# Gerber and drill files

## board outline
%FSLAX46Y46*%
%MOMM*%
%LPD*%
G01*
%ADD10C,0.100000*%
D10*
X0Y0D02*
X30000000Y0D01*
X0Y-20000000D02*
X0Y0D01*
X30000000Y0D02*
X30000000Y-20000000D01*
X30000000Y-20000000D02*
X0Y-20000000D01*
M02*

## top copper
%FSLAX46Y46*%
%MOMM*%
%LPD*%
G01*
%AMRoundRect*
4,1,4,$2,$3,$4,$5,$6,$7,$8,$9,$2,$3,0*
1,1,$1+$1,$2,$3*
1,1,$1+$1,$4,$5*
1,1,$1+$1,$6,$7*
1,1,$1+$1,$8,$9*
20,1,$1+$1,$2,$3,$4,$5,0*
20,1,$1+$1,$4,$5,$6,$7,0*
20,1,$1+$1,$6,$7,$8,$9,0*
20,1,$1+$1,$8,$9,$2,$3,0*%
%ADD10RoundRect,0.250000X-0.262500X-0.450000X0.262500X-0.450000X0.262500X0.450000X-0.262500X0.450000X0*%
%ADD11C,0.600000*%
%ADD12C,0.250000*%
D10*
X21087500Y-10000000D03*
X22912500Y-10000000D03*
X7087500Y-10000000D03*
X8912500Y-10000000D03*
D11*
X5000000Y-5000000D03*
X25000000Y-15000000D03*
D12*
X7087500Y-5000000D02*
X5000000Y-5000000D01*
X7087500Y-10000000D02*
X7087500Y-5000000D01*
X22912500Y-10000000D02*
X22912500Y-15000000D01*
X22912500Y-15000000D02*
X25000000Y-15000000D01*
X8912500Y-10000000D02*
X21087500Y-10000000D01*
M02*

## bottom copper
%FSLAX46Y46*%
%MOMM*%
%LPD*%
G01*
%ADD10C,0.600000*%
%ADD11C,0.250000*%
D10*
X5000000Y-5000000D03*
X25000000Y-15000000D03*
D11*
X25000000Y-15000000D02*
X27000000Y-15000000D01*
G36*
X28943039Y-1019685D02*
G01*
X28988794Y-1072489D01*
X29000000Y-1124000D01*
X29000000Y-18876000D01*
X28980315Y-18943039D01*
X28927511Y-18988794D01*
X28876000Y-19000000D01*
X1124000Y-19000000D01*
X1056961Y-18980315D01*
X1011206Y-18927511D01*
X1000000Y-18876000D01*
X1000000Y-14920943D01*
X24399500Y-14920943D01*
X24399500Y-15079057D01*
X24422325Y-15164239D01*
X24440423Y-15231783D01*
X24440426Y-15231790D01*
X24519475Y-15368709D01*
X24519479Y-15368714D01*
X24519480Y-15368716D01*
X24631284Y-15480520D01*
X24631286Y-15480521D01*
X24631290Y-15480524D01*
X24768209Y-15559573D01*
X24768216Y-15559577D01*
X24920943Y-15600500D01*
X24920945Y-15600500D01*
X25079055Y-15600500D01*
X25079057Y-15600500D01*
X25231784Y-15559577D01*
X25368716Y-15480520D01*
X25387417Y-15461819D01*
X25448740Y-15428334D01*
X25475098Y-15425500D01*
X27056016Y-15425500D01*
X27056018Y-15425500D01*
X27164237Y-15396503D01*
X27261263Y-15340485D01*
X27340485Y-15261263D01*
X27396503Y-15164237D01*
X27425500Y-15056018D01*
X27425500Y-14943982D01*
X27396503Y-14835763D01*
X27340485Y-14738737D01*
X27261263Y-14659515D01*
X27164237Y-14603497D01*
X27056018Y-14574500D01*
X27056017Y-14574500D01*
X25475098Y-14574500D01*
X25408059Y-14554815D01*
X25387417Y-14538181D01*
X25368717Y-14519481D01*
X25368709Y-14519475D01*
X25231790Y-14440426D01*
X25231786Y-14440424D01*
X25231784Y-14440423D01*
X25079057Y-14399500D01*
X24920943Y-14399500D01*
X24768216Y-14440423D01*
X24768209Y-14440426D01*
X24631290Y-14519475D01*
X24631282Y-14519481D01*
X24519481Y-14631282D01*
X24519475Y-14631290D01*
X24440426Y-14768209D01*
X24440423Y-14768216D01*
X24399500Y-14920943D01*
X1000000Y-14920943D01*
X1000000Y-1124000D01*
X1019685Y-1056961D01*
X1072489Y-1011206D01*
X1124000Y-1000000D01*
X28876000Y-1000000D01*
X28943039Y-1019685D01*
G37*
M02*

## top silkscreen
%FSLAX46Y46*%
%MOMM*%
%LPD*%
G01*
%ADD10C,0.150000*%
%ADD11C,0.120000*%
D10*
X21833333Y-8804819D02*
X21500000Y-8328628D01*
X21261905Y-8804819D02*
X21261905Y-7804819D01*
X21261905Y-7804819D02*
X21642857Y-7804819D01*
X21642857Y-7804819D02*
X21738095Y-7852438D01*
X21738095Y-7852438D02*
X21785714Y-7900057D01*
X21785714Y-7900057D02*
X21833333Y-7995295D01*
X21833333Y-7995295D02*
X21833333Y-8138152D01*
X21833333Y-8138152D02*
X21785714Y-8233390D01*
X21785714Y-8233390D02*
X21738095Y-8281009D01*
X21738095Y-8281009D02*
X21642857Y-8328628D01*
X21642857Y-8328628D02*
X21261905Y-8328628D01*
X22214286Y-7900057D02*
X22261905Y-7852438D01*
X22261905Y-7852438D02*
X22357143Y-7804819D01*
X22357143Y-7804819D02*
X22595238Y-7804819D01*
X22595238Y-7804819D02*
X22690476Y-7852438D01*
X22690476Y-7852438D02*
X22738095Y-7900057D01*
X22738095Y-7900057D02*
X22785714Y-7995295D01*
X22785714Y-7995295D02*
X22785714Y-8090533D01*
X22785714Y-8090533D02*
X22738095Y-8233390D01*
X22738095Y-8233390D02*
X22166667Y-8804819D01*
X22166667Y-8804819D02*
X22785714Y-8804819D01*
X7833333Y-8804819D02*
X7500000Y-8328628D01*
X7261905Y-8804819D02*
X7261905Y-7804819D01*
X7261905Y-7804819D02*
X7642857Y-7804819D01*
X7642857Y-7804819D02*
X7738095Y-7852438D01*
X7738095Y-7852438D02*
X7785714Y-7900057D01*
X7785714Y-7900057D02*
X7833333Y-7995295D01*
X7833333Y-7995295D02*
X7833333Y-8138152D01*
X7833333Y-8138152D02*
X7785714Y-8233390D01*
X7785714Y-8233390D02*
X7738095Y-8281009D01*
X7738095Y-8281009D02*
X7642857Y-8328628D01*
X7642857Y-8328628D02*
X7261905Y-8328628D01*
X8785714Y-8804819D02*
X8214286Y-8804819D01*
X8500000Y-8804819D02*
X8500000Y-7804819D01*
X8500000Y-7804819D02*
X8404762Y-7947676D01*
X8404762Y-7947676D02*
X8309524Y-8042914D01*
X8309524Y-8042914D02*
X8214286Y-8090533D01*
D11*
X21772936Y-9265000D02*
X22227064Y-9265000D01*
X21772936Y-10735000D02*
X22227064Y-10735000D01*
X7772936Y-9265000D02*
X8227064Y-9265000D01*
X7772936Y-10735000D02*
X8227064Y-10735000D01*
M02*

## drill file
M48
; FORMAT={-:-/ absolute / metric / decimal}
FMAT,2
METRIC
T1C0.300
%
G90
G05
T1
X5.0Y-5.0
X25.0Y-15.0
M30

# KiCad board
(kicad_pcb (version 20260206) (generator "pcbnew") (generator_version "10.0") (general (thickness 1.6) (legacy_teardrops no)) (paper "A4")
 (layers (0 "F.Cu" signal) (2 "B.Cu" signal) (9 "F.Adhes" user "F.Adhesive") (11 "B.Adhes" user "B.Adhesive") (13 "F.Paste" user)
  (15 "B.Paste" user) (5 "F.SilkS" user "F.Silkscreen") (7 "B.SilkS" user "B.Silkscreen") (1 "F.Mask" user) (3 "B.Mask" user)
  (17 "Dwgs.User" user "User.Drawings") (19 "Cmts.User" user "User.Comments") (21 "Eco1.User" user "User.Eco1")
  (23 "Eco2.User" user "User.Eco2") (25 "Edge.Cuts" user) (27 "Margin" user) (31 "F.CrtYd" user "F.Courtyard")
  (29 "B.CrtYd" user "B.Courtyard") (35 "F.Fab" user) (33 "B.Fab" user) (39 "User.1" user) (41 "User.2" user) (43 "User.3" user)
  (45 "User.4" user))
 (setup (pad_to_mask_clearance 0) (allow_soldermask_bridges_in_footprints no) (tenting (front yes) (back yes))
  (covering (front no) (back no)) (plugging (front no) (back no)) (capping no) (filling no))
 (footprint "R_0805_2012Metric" (layer "F.Cu") (at 22 10)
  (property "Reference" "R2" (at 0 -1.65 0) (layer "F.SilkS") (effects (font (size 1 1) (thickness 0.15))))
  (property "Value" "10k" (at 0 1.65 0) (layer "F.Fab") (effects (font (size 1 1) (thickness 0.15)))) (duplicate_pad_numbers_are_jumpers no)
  (fp_line (start -0.227064 -0.735) (end 0.227064 -0.735) (stroke (width 0.12) (type solid)) (layer "F.SilkS"))
  (fp_line (start -0.227064 0.735) (end 0.227064 0.735) (stroke (width 0.12) (type solid)) (layer "F.SilkS"))
  (pad "1" smd roundrect (at -0.9125 0) (size 1.025 1.4) (layers "F.Cu" "F.Mask" "F.Paste") (roundrect_rratio 0.243902) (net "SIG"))
  (pad "2" smd roundrect (at 0.9125 0) (size 1.025 1.4) (layers "F.Cu" "F.Mask" "F.Paste") (roundrect_rratio 0.243902) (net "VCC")))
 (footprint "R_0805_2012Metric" (layer "F.Cu") (at 8 10)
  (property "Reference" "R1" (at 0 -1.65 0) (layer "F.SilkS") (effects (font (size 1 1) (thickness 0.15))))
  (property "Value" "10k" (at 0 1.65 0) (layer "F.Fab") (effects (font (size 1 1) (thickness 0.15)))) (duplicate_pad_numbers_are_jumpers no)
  (fp_line (start -0.227064 -0.735) (end 0.227064 -0.735) (stroke (width 0.12) (type solid)) (layer "F.SilkS"))
  (fp_line (start -0.227064 0.735) (end 0.227064 0.735) (stroke (width 0.12) (type solid)) (layer "F.SilkS"))
  (pad "1" smd roundrect (at -0.9125 0) (size 1.025 1.4) (layers "F.Cu" "F.Mask" "F.Paste") (roundrect_rratio 0.243902) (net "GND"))
  (pad "2" smd roundrect (at 0.9125 0) (size 1.025 1.4) (layers "F.Cu" "F.Mask" "F.Paste") (roundrect_rratio 0.243902) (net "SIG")))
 (gr_line (start 0 0) (end 30 0) (stroke (width 0.1) (type default)) (layer "Edge.Cuts"))
 (gr_line (start 0 20) (end 0 0) (stroke (width 0.1) (type default)) (layer "Edge.Cuts"))
 (gr_line (start 30 0) (end 30 20) (stroke (width 0.1) (type default)) (layer "Edge.Cuts"))
 (gr_line (start 30 20) (end 0 20) (stroke (width 0.1) (type default)) (layer "Edge.Cuts"))
 (segment (start 7.0875 5) (end 5 5) (width 0.25) (layer "F.Cu") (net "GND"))
 (segment (start 7.0875 10) (end 7.0875 5) (width 0.25) (layer "F.Cu") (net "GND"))
 (via (at 5 5) (size 0.6) (drill 0.3) (layers "F.Cu" "B.Cu") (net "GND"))
 (segment (start 22.9125 10) (end 22.9125 15) (width 0.25) (layer "F.Cu") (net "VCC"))
 (segment (start 22.9125 15) (end 25 15) (width 0.25) (layer "F.Cu") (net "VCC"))
 (via (at 25 15) (size 0.6) (drill 0.3) (layers "F.Cu" "B.Cu") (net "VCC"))
 (segment (start 25 15) (end 27 15) (width 0.25) (layer "B.Cu") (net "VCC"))
 (segment (start 8.9125 10) (end 21.0875 10) (width 0.25) (layer "F.Cu") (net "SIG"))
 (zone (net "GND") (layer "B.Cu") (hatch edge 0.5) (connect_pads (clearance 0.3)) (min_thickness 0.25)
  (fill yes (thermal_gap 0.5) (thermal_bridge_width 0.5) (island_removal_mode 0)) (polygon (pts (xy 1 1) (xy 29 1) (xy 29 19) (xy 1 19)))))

